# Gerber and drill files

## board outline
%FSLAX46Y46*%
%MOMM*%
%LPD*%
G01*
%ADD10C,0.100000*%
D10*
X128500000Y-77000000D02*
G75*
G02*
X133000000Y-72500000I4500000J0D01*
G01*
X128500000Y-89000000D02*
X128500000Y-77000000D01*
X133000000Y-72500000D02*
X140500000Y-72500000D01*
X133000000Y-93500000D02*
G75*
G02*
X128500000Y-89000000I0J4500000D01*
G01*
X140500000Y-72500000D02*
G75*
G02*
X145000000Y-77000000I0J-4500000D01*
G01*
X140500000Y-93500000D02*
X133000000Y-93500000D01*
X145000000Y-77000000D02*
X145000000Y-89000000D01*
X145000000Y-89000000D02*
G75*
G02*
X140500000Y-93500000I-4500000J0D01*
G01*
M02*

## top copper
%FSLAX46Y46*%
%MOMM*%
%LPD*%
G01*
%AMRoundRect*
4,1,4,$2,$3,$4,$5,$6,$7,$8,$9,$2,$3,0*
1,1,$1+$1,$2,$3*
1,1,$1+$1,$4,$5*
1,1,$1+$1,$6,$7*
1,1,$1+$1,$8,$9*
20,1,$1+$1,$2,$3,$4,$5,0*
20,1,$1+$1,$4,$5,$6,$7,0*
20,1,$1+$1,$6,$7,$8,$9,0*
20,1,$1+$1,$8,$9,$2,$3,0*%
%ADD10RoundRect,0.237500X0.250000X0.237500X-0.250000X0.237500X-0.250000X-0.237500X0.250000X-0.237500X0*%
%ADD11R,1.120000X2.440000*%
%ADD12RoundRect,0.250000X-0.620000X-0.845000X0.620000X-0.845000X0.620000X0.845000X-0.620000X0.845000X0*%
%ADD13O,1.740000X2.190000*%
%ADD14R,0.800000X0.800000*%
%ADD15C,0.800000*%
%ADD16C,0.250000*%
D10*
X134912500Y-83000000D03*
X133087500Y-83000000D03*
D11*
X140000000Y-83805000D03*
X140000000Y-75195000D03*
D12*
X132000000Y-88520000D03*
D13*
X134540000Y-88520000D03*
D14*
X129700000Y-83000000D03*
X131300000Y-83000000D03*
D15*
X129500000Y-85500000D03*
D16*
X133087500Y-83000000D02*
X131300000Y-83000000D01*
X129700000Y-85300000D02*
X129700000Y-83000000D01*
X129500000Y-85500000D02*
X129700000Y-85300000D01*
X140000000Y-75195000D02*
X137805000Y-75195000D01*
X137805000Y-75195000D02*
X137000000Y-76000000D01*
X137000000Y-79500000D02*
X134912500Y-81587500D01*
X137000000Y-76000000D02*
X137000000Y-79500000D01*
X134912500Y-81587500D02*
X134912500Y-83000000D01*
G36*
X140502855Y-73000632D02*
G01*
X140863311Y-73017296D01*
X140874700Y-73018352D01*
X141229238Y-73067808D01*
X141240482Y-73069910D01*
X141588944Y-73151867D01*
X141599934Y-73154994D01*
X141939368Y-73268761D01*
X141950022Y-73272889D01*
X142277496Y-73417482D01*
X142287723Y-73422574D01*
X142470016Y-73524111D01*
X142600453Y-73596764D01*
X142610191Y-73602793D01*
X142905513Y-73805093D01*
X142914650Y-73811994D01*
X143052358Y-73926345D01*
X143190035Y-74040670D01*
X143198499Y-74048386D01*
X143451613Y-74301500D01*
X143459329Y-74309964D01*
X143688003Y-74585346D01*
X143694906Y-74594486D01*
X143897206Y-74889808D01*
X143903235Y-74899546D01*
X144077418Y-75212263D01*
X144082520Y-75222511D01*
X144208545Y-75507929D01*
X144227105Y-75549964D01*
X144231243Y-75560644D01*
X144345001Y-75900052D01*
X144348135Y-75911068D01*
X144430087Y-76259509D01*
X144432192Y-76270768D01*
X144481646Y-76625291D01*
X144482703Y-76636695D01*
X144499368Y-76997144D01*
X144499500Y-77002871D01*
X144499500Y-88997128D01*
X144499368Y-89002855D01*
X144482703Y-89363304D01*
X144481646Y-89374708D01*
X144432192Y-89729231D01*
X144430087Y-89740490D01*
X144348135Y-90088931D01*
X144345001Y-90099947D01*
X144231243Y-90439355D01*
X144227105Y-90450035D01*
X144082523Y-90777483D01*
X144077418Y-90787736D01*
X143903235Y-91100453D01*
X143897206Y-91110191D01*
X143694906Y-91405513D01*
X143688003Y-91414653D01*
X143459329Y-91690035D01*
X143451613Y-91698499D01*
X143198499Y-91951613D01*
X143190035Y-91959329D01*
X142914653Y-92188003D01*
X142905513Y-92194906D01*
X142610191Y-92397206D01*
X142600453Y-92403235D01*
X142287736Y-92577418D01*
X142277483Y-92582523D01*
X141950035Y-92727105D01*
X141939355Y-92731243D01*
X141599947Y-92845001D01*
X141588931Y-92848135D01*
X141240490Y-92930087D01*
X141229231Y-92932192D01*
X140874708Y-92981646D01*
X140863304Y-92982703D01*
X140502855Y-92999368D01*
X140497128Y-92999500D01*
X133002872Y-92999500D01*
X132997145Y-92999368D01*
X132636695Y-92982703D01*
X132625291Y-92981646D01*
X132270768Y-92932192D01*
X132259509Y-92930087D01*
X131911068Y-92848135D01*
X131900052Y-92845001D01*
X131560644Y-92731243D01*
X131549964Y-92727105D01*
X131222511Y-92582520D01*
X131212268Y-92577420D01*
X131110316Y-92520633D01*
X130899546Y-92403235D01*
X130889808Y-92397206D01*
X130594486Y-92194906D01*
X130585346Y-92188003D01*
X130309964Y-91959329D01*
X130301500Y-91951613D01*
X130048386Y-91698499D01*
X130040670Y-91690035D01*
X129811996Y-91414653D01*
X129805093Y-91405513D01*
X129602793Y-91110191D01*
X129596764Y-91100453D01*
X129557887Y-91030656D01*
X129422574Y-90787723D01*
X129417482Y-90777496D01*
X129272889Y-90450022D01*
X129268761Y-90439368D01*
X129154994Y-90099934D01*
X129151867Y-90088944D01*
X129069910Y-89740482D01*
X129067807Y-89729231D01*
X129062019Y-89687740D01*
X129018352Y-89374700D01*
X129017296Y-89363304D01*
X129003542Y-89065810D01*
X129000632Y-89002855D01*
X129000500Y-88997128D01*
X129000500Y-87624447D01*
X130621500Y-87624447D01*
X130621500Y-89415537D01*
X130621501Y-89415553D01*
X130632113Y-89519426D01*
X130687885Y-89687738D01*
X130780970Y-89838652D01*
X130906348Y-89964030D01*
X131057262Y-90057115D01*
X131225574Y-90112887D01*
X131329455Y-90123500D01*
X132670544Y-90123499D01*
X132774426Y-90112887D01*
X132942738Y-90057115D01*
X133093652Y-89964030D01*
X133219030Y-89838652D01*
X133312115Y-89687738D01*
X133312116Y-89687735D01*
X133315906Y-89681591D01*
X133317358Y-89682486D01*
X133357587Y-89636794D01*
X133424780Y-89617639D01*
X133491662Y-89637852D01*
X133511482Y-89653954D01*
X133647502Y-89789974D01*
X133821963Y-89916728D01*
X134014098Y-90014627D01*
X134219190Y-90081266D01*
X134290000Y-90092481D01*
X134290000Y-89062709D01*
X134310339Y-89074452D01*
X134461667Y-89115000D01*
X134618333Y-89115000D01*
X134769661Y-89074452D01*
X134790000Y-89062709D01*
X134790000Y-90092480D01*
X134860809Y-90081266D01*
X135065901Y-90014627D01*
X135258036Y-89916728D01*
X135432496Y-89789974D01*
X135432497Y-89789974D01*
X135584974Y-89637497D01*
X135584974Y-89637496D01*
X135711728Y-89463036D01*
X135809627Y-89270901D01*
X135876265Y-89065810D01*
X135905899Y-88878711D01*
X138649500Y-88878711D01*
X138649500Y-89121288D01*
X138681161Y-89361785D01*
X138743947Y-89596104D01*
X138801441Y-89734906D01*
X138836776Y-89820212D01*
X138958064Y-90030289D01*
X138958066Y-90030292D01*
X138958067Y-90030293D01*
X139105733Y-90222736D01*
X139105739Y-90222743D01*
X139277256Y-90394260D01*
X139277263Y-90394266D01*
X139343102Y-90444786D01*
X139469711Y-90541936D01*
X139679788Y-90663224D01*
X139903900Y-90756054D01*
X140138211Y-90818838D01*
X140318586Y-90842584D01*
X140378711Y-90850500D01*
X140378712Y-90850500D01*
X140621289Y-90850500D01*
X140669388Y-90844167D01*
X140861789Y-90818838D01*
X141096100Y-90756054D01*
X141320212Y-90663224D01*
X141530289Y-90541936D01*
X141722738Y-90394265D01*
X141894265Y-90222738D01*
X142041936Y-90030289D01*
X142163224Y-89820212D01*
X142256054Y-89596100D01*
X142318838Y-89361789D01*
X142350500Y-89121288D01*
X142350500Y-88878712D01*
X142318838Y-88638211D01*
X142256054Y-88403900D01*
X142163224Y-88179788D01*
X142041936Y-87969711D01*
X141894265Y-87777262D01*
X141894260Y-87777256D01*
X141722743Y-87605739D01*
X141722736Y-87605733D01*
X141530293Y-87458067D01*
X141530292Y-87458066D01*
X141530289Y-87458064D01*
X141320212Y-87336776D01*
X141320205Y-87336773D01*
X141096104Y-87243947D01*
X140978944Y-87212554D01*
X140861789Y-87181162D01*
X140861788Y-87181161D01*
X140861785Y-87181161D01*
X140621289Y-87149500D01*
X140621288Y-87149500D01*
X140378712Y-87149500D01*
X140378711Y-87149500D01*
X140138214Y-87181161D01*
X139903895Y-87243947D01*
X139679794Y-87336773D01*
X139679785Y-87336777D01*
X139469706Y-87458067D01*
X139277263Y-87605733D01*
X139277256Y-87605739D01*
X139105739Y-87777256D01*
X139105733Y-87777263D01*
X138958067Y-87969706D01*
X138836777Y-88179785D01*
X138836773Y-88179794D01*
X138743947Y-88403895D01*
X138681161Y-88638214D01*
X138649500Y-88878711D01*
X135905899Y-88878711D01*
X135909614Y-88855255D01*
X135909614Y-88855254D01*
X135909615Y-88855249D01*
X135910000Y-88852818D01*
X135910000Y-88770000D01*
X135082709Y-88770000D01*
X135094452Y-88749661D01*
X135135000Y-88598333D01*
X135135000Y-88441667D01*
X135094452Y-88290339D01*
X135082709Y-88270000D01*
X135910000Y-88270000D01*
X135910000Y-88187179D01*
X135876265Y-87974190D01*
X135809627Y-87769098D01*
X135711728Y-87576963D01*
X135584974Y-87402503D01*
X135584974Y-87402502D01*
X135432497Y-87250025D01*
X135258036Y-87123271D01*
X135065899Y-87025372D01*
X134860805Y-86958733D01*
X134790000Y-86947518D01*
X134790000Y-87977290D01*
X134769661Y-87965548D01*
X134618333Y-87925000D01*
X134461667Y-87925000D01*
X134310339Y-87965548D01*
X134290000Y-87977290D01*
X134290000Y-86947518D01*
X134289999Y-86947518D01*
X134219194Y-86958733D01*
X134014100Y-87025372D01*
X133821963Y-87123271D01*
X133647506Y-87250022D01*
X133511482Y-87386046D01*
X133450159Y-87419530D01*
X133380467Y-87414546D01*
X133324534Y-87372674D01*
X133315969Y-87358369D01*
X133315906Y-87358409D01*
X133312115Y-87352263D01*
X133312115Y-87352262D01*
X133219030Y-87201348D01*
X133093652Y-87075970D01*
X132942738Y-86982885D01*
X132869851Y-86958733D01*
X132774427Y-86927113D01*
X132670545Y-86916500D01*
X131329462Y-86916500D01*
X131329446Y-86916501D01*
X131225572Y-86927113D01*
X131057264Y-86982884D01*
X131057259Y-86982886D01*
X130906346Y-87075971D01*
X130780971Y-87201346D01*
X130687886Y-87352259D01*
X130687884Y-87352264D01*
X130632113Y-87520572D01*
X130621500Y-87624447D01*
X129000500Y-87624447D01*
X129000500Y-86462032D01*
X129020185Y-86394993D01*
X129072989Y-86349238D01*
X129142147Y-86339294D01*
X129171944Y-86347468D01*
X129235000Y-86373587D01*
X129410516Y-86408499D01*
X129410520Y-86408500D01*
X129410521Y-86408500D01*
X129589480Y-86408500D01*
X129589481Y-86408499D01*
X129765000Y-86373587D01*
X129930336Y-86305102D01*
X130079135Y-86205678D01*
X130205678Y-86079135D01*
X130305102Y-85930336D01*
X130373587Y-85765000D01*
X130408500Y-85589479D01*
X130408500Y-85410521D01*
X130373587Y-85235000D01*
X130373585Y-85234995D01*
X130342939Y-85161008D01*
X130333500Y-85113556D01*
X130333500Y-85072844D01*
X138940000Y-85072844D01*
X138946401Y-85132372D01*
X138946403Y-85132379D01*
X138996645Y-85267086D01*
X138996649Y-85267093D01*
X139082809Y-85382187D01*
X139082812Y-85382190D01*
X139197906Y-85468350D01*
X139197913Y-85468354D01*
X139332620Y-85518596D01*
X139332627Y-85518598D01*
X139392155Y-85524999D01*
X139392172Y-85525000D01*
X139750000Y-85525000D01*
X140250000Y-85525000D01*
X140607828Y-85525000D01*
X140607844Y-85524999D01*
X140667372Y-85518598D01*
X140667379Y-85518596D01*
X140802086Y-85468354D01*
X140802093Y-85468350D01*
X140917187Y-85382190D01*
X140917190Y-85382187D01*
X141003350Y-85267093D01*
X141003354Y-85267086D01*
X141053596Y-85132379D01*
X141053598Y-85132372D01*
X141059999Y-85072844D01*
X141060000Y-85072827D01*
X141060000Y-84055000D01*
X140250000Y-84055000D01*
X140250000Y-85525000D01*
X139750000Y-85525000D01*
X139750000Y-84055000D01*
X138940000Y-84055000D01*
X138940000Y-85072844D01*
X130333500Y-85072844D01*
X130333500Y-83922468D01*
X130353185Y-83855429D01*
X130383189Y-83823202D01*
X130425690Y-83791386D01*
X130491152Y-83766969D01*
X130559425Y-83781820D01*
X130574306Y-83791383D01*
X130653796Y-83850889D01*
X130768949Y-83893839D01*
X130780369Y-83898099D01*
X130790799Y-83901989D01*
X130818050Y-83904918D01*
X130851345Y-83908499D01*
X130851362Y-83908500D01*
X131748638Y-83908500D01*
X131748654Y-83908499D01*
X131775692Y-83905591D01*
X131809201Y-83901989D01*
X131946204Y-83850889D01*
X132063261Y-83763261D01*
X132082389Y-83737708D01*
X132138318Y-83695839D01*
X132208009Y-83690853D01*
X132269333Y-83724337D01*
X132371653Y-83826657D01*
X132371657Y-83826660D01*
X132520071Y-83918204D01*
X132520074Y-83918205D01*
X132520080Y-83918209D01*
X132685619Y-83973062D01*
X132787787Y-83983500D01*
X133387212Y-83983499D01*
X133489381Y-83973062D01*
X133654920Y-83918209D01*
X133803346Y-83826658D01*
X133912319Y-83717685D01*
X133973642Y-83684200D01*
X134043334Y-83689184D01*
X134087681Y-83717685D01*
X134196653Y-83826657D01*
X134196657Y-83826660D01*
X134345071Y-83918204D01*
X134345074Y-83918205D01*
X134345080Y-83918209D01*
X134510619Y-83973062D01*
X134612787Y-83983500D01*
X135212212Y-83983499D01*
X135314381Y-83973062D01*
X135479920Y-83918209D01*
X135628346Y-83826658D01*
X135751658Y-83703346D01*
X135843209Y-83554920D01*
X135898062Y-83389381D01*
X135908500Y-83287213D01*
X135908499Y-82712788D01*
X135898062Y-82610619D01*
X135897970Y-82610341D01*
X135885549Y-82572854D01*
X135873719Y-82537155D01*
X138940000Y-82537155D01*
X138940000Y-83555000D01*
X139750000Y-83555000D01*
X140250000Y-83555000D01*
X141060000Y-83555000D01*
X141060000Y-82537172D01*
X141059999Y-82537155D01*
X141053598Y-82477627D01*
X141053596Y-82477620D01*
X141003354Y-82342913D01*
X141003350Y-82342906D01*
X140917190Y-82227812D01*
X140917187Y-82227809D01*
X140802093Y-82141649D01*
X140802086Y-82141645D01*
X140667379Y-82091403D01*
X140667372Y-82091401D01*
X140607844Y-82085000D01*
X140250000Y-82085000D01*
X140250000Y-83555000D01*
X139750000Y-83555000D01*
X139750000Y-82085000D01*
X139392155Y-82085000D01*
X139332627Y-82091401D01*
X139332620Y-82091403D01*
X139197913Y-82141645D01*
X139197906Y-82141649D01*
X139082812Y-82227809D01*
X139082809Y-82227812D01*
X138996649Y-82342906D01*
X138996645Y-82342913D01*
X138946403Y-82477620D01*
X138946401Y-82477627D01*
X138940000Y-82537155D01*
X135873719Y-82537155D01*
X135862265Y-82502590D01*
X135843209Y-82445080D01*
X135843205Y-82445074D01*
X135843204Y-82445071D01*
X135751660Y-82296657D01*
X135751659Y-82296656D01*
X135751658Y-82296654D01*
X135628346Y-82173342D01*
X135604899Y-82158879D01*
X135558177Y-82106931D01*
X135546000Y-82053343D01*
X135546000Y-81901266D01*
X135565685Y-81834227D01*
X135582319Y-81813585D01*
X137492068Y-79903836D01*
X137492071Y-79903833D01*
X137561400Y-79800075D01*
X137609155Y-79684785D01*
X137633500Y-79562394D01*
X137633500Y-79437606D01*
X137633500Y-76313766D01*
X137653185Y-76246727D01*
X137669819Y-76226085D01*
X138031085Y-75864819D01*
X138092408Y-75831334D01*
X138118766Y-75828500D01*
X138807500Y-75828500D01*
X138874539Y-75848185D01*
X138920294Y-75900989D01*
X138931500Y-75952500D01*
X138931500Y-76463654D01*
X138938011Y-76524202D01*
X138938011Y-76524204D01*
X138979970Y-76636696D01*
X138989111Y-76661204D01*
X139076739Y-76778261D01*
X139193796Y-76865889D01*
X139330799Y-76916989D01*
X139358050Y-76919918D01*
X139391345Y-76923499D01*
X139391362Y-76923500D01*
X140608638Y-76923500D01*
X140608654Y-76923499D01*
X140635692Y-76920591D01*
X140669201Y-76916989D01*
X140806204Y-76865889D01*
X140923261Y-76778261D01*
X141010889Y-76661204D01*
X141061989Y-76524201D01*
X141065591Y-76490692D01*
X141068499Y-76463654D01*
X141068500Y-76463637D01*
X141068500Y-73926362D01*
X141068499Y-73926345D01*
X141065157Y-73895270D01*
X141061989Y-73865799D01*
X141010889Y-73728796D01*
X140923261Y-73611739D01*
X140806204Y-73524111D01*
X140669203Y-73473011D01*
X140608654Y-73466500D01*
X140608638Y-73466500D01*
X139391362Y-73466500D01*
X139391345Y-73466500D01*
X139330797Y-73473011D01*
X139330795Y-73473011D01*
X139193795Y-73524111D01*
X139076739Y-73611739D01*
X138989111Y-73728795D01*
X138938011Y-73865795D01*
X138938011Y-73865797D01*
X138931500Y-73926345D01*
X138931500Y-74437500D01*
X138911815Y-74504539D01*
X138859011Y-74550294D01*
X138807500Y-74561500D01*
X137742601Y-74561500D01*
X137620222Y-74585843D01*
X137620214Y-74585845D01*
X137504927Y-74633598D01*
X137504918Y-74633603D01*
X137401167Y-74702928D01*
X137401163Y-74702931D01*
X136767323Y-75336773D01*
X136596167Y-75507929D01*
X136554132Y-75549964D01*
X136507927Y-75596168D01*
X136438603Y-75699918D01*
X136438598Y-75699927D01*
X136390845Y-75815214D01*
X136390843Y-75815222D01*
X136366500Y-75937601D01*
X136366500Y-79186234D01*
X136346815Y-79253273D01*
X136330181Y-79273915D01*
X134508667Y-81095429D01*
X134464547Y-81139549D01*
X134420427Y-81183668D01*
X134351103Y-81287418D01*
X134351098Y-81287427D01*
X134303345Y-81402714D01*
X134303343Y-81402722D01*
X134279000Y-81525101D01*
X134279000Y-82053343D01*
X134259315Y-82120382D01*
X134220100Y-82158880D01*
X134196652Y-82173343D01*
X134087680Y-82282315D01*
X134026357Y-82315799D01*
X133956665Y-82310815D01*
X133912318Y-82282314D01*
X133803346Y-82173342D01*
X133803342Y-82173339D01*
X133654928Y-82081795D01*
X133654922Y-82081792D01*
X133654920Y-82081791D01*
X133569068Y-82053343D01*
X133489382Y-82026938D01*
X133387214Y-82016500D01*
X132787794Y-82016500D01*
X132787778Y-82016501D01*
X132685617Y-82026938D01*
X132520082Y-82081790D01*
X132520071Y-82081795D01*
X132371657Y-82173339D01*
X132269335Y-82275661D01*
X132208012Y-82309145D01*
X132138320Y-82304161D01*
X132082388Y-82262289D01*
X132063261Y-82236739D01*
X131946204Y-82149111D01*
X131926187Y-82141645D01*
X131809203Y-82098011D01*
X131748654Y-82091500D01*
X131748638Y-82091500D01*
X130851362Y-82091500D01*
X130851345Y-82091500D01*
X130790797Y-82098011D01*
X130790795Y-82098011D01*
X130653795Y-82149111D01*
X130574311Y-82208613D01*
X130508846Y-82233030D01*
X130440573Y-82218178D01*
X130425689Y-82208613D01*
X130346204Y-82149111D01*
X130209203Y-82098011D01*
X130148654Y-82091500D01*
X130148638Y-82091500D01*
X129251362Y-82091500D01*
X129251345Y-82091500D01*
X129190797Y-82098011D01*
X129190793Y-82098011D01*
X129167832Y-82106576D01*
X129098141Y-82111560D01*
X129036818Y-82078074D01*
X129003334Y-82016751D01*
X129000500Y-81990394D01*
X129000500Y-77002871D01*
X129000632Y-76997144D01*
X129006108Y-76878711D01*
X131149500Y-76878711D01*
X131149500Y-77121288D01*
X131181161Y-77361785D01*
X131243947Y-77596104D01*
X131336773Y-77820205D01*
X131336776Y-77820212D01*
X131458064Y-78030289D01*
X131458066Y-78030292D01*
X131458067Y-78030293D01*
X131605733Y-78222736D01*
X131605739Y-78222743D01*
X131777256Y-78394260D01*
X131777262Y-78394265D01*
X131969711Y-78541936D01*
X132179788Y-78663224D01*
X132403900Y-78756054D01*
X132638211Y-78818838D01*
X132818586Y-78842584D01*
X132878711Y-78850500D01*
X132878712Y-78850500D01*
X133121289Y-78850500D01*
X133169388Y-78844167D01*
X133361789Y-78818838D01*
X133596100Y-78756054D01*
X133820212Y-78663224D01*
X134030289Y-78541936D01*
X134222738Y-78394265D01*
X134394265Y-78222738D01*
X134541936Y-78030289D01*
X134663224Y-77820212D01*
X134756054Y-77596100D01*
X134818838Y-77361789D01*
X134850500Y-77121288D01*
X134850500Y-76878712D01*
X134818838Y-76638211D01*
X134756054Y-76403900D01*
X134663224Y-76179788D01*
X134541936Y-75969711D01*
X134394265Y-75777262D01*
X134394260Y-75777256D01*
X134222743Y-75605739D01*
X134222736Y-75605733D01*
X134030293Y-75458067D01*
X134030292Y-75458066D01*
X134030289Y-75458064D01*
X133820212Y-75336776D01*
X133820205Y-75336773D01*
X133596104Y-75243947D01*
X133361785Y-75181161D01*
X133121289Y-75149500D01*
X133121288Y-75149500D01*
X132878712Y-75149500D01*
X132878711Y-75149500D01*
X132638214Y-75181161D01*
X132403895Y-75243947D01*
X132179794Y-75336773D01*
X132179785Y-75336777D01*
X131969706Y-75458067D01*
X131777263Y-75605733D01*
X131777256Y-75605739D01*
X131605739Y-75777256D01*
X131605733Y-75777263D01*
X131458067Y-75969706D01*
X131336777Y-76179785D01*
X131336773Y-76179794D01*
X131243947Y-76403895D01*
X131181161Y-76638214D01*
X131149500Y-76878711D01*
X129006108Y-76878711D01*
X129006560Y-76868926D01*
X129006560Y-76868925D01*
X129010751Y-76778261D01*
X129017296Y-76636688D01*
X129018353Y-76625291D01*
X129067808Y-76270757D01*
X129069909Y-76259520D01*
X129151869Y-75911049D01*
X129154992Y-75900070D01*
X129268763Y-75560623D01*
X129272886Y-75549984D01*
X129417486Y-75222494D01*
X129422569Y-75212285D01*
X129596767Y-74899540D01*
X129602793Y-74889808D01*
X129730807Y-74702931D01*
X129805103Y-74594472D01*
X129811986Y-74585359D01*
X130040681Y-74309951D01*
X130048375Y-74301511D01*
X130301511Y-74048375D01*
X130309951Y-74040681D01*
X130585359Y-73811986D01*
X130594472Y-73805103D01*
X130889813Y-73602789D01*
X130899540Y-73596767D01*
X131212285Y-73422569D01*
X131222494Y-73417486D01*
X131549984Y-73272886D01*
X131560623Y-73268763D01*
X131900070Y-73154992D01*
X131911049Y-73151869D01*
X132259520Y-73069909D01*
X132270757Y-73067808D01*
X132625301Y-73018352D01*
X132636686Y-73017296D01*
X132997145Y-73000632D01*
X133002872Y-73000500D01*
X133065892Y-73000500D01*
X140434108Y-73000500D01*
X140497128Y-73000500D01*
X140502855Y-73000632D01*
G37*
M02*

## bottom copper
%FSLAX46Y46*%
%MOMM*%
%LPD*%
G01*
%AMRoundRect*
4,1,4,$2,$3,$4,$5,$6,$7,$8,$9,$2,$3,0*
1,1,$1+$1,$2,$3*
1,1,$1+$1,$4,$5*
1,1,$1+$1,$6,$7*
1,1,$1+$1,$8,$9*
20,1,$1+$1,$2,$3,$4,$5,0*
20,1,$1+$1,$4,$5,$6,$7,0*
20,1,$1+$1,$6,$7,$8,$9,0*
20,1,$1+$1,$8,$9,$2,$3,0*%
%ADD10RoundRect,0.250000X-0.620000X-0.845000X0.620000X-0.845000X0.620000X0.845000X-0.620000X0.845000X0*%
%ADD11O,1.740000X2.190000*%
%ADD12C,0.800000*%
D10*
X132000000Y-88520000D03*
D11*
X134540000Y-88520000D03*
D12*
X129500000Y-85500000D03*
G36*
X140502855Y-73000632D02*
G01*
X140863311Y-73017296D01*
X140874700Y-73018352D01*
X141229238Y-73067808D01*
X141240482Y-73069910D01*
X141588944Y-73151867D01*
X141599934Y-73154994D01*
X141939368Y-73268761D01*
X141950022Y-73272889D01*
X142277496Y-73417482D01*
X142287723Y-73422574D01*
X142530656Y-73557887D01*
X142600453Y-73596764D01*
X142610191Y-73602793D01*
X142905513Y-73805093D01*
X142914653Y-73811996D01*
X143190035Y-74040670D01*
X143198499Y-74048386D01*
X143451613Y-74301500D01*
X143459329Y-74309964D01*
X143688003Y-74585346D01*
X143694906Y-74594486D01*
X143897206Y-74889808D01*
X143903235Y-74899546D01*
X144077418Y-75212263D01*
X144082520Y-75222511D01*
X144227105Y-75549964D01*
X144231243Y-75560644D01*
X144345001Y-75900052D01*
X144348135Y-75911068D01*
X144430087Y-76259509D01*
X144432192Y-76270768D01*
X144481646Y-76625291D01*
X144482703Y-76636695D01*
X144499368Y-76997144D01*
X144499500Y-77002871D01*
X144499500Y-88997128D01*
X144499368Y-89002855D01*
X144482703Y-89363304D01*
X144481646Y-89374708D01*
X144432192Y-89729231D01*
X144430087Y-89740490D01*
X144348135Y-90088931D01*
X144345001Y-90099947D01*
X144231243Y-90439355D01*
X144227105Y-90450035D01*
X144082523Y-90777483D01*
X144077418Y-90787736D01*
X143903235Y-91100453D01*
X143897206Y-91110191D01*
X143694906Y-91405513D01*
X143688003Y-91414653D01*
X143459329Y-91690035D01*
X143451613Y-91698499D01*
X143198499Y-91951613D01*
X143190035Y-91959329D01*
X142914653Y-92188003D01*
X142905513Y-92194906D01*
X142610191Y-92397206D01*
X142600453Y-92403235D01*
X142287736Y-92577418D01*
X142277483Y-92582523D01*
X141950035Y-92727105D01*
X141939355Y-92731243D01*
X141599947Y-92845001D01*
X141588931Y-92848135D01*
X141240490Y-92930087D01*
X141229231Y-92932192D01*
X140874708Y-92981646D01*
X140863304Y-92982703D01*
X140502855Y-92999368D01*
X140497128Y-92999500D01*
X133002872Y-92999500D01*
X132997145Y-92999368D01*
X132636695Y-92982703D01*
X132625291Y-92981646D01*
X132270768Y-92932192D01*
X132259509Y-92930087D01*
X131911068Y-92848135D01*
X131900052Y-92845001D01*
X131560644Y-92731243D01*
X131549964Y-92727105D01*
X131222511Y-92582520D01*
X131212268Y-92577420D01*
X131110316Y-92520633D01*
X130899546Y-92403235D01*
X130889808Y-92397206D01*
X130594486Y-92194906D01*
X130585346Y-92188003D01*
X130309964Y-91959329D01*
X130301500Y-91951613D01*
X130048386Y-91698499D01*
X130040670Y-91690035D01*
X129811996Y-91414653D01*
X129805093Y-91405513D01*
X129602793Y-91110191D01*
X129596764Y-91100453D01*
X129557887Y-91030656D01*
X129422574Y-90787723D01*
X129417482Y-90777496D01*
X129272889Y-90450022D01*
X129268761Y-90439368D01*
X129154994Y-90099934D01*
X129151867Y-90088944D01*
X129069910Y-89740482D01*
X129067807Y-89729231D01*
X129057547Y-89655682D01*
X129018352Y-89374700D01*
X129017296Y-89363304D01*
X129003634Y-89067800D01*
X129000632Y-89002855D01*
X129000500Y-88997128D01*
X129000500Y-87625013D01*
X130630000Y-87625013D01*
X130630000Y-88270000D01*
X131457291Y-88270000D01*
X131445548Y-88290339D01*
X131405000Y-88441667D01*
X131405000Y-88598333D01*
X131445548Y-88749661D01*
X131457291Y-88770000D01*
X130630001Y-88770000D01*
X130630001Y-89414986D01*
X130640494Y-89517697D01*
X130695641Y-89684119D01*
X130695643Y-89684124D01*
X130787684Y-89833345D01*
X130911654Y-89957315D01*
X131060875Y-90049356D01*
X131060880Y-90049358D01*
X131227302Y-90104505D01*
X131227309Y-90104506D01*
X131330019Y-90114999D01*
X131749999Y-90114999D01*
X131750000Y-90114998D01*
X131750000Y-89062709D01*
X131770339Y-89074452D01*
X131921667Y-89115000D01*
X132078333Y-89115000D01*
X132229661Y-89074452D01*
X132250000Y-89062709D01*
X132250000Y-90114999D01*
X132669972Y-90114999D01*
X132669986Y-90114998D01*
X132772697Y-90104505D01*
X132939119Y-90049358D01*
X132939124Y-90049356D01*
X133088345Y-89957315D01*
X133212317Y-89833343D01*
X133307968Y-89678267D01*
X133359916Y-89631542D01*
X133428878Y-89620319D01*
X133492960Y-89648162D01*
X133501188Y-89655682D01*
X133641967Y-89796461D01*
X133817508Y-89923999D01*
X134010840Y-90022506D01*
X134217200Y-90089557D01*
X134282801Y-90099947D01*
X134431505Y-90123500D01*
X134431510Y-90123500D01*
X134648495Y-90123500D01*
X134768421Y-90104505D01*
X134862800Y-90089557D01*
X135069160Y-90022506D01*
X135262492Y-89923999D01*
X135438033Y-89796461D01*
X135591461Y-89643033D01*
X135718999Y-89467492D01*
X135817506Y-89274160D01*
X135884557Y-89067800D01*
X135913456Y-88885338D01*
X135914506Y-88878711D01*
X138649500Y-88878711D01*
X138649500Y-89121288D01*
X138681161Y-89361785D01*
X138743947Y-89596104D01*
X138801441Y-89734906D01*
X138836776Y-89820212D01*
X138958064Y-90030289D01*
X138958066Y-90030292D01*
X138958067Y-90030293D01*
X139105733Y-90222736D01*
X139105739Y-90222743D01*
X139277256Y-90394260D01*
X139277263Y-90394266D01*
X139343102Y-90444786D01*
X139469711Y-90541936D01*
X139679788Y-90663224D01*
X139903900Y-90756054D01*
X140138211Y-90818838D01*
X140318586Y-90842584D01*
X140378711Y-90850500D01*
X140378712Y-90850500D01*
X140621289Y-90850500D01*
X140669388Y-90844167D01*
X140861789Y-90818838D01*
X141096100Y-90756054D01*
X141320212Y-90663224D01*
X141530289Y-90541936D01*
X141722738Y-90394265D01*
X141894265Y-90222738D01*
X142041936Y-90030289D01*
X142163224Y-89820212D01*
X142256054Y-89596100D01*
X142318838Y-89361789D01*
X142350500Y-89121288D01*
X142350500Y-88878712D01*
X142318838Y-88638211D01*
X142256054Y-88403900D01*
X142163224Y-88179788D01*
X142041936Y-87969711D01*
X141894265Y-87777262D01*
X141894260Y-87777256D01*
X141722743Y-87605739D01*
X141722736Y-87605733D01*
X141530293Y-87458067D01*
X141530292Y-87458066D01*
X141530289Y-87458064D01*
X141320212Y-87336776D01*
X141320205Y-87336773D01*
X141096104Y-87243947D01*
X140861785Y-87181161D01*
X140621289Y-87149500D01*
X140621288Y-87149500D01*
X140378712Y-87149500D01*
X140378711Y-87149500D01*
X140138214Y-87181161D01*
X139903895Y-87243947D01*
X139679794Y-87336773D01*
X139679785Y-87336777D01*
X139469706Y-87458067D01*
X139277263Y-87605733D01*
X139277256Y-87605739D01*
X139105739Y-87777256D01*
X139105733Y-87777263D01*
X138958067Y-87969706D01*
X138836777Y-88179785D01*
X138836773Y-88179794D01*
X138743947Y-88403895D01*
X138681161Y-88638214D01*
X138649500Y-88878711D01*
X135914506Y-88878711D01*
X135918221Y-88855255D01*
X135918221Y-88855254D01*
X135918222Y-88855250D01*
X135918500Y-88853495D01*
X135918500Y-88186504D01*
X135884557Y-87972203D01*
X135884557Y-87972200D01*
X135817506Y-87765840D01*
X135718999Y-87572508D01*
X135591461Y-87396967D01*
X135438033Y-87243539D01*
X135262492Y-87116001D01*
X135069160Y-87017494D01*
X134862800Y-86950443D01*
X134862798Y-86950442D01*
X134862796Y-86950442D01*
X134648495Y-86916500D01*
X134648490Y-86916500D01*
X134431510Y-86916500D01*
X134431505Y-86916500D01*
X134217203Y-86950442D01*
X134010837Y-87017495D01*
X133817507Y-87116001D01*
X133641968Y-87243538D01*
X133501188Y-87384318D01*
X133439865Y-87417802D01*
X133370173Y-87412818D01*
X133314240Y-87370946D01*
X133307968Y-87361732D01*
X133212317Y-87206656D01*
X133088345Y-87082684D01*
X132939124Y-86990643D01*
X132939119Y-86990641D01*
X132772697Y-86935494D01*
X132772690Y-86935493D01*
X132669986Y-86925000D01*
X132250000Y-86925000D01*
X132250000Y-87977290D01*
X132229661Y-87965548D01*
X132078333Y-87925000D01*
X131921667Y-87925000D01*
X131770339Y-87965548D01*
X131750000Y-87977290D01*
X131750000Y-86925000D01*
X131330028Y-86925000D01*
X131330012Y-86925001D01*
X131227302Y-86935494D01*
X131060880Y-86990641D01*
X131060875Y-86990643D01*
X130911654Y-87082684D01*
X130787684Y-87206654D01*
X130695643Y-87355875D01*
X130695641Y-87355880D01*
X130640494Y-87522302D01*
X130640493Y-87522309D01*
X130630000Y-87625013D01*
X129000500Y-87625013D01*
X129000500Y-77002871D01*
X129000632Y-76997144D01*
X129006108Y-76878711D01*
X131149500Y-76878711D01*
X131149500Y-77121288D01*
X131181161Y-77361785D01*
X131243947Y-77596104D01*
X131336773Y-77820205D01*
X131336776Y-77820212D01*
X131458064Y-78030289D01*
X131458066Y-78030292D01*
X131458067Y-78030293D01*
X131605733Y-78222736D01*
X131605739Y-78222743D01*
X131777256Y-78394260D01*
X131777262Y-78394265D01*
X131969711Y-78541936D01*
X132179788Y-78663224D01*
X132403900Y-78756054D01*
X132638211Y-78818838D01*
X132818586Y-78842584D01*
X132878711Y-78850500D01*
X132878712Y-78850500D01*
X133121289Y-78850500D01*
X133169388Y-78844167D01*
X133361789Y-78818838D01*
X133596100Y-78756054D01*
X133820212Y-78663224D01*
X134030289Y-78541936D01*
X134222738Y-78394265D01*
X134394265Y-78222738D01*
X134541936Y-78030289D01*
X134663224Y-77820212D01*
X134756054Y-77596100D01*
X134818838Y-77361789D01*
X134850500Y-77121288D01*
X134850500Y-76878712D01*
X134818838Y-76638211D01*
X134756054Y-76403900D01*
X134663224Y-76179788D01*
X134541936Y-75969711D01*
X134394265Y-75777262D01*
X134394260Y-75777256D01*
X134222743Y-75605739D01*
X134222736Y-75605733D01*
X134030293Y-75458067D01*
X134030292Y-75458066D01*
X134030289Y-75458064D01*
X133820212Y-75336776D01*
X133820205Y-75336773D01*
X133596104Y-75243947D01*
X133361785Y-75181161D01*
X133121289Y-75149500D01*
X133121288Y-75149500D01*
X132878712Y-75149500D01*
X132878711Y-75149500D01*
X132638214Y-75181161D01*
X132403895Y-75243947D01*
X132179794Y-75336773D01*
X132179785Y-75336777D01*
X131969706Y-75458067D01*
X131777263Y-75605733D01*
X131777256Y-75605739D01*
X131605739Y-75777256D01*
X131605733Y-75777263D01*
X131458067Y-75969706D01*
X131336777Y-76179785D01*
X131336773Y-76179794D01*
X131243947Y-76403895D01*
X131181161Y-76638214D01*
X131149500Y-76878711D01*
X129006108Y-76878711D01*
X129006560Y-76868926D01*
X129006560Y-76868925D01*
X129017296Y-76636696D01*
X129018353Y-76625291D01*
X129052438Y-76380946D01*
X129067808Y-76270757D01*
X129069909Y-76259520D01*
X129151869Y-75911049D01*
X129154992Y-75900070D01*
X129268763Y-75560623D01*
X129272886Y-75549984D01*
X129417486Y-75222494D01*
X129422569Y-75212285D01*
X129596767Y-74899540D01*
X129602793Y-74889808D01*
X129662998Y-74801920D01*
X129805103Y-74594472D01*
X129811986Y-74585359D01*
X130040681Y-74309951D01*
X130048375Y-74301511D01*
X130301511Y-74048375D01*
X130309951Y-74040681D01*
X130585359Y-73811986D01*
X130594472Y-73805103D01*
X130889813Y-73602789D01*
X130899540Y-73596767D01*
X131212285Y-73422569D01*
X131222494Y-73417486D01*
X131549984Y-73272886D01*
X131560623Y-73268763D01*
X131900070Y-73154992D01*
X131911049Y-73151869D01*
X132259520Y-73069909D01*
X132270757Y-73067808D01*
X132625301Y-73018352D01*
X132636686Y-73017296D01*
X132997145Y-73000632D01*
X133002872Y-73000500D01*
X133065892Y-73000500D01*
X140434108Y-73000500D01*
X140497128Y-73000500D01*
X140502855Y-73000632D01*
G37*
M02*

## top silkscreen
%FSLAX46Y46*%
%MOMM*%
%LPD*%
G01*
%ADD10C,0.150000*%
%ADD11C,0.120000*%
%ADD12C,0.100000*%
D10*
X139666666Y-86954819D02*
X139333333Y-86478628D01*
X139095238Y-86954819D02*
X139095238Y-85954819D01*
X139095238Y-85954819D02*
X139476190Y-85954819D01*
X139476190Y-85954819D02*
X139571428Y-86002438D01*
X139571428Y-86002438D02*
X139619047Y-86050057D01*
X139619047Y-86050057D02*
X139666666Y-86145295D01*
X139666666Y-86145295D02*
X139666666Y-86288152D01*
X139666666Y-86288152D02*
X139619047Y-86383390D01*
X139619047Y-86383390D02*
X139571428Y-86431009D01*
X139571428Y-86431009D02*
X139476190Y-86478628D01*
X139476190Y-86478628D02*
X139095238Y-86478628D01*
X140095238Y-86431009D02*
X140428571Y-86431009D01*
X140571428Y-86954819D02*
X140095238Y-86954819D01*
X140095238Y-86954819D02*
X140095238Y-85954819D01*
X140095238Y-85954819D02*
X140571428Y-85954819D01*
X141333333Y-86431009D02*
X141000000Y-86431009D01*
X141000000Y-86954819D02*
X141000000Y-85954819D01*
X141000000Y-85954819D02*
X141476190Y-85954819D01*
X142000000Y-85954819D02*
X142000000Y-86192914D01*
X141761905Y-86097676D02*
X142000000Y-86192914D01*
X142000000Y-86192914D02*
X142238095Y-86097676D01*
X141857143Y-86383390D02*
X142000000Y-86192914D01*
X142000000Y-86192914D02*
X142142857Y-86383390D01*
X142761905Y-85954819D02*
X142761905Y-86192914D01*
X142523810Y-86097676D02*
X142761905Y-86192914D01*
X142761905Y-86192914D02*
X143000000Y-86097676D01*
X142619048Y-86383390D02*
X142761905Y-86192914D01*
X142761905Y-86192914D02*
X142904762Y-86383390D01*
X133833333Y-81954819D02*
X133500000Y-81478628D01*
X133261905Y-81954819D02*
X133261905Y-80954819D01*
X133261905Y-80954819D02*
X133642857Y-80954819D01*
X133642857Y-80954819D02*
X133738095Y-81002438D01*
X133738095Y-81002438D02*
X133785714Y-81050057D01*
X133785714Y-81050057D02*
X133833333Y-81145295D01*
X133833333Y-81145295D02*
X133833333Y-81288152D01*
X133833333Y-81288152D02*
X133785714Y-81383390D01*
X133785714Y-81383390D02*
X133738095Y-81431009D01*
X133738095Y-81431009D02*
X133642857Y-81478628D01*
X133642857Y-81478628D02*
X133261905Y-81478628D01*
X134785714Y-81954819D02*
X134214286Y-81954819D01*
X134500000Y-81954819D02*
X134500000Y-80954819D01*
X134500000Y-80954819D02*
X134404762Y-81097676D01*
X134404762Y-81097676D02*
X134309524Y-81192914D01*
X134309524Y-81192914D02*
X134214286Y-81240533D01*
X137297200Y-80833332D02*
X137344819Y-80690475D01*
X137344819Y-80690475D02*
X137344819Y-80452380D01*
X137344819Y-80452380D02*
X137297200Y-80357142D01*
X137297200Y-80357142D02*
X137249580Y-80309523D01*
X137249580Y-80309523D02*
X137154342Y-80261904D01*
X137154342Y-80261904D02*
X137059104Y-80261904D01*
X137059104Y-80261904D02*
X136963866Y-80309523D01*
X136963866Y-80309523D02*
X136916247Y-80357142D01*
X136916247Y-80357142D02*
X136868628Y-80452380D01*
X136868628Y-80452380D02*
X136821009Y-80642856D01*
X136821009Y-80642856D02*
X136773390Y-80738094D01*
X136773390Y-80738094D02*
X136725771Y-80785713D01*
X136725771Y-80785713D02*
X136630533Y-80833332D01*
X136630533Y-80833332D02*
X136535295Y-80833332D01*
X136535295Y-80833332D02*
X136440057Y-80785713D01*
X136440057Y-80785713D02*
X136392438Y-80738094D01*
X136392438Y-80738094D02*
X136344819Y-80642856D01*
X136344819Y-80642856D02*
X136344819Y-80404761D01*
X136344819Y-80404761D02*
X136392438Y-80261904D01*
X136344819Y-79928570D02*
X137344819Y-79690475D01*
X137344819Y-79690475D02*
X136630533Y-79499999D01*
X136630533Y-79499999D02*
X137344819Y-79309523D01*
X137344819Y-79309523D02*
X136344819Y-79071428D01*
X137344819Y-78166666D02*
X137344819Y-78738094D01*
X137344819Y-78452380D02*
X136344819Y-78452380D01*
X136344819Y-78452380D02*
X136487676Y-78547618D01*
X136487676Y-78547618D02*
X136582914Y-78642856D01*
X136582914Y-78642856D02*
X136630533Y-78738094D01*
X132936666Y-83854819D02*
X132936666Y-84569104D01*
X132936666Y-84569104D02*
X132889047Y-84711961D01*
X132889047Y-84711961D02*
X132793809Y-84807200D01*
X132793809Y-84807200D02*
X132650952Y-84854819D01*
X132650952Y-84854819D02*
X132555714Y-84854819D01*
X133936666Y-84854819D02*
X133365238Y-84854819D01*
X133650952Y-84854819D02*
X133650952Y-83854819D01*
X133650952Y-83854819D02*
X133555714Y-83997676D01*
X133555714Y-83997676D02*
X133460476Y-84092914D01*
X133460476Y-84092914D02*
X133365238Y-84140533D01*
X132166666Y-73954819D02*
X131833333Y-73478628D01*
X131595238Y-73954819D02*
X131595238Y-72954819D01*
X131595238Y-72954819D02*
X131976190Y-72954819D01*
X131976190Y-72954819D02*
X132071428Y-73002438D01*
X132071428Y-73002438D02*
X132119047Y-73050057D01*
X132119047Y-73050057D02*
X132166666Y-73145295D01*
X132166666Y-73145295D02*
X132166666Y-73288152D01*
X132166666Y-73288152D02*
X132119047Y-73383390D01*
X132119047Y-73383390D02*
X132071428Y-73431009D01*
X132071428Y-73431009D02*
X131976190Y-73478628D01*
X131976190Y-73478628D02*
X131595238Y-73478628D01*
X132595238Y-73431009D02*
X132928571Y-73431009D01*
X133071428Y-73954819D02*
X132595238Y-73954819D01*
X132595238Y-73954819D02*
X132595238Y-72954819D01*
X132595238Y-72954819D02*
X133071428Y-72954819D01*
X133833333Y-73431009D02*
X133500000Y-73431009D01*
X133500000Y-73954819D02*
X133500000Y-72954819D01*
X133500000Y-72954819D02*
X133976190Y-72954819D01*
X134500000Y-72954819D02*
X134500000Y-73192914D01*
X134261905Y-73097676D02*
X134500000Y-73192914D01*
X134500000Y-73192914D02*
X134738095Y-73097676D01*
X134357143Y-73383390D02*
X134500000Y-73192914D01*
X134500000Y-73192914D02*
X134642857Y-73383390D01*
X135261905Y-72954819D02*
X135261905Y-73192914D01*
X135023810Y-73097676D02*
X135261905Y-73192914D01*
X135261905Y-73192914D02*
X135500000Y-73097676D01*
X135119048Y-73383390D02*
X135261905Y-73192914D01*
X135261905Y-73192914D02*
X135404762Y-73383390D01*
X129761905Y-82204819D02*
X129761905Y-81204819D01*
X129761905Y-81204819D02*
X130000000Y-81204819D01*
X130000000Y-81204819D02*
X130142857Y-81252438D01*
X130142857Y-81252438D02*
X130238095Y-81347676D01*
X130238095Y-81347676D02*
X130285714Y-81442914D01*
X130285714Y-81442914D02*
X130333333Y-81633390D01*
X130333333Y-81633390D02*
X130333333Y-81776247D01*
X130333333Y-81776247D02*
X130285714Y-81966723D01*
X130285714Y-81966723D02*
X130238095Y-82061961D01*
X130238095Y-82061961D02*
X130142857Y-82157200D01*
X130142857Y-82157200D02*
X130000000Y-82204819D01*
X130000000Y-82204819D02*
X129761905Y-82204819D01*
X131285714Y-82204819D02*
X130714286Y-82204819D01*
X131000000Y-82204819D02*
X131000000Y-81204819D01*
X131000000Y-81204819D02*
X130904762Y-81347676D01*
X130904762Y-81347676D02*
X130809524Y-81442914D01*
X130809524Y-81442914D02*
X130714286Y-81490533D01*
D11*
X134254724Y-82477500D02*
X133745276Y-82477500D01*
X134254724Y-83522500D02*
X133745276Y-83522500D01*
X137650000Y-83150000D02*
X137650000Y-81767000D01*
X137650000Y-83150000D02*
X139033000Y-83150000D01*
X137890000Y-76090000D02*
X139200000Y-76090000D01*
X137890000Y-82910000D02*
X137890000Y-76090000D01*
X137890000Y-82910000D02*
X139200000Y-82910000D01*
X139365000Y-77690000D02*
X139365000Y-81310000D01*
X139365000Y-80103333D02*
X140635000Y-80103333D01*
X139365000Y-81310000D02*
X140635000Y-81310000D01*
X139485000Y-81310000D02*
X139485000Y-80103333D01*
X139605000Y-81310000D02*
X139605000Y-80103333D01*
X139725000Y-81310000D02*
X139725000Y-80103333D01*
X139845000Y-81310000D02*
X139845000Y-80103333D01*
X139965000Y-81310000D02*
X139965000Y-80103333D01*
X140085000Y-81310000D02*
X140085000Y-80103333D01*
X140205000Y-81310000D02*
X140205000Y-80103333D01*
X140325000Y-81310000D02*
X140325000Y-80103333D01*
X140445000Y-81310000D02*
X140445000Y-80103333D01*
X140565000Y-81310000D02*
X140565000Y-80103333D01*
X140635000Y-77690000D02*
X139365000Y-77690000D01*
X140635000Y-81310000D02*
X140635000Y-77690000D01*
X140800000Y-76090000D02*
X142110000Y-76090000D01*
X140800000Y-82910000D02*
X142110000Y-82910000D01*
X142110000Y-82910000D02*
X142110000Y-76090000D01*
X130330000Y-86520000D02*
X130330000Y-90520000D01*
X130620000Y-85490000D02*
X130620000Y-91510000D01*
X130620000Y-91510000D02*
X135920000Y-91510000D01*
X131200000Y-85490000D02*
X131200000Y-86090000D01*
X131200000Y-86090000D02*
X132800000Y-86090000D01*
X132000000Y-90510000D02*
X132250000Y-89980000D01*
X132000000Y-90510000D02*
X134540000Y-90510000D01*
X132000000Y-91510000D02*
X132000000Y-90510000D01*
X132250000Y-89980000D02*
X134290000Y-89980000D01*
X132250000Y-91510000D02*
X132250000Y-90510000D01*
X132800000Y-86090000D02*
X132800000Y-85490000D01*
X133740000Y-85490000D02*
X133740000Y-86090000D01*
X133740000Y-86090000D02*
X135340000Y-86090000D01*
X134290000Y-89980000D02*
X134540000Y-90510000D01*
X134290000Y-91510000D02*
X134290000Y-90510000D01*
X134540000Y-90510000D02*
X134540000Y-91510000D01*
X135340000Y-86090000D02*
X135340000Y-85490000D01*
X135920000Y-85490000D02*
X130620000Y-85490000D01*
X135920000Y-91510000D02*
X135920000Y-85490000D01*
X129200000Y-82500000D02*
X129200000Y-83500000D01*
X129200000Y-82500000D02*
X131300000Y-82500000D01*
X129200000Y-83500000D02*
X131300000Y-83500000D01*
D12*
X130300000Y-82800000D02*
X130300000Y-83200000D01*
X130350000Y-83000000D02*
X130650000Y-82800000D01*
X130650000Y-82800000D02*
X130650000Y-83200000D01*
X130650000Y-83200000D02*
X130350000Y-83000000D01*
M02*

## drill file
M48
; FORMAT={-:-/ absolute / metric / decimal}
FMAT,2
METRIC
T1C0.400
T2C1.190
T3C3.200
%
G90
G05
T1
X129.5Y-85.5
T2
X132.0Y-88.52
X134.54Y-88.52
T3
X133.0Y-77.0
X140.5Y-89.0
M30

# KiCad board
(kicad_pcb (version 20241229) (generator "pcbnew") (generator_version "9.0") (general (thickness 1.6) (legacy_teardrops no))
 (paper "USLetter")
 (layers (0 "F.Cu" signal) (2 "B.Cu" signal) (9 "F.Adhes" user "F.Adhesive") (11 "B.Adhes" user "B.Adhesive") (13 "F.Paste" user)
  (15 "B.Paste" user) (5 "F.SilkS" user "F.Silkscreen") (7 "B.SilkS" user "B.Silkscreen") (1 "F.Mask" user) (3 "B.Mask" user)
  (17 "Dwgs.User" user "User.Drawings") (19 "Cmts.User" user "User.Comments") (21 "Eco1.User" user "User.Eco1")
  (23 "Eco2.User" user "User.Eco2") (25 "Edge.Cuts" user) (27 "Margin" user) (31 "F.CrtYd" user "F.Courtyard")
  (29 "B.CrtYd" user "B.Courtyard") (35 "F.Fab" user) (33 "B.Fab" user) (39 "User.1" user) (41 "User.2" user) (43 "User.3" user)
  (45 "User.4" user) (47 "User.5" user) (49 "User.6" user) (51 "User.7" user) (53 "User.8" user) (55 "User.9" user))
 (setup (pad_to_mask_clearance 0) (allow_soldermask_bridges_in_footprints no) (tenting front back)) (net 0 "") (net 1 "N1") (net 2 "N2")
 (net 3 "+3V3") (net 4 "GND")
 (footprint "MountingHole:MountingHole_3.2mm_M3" (layer "F.Cu") (at 140.5 89)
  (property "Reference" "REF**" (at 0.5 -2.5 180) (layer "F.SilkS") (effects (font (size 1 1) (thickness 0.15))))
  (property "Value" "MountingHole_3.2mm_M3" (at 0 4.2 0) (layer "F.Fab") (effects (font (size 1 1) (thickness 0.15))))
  (pad "" np_thru_hole circle (at 0 0) (size 3.2 3.2) (drill 3.2) (layers "*.Cu" "*.Mask")))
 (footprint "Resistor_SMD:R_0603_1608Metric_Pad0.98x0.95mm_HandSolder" (layer "F.Cu") (at 134 83 180)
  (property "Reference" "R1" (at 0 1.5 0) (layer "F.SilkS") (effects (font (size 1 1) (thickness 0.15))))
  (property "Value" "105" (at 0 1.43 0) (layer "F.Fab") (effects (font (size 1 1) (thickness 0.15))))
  (fp_line (start -0.254724 0.5225) (end 0.254724 0.5225) (stroke (width 0.12) (type solid)) (layer "F.SilkS"))
  (fp_line (start -0.254724 -0.5225) (end 0.254724 -0.5225) (stroke (width 0.12) (type solid)) (layer "F.SilkS"))
  (pad "1" smd roundrect (at -0.9125 0 180) (size 0.975 0.95) (layers "F.Cu" "F.Mask" "F.Paste") (roundrect_rratio 0.25) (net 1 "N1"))
  (pad "2" smd roundrect (at 0.9125 0 180) (size 0.975 0.95) (layers "F.Cu" "F.Mask" "F.Paste") (roundrect_rratio 0.25) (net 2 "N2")))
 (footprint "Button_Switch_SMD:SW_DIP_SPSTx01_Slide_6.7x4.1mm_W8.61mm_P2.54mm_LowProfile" (layer "F.Cu") (at 140 79.5 90)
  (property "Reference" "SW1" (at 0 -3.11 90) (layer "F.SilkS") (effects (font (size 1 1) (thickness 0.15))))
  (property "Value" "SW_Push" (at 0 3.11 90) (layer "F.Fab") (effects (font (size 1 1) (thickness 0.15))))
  (fp_line (start -3.65 -2.35) (end -2.267 -2.35) (stroke (width 0.12) (type solid)) (layer "F.SilkS"))
  (fp_line (start -3.65 -2.35) (end -3.65 -0.967) (stroke (width 0.12) (type solid)) (layer "F.SilkS"))
  (fp_line (start 3.41 -2.11) (end 3.41 -0.8) (stroke (width 0.12) (type solid)) (layer "F.SilkS"))
  (fp_line (start -3.41 -2.11) (end 3.41 -2.11) (stroke (width 0.12) (type solid)) (layer "F.SilkS"))
  (fp_line (start -3.41 -2.11) (end -3.41 -0.8) (stroke (width 0.12) (type solid)) (layer "F.SilkS"))
  (fp_line (start 1.81 -0.635) (end -1.81 -0.635) (stroke (width 0.12) (type solid)) (layer "F.SilkS"))
  (fp_line (start -0.603333 -0.635) (end -0.603333 0.635) (stroke (width 0.12) (type solid)) (layer "F.SilkS"))
  (fp_line (start -1.81 -0.635) (end -1.81 0.635) (stroke (width 0.12) (type solid)) (layer "F.SilkS"))
  (fp_line (start -1.81 -0.515) (end -0.603333 -0.515) (stroke (width 0.12) (type solid)) (layer "F.SilkS"))
  (fp_line (start -1.81 -0.395) (end -0.603333 -0.395) (stroke (width 0.12) (type solid)) (layer "F.SilkS"))
  (fp_line (start -1.81 -0.275) (end -0.603333 -0.275) (stroke (width 0.12) (type solid)) (layer "F.SilkS"))
  (fp_line (start -1.81 -0.155) (end -0.603333 -0.155) (stroke (width 0.12) (type solid)) (layer "F.SilkS"))
  (fp_line (start -1.81 -0.035) (end -0.603333 -0.035) (stroke (width 0.12) (type solid)) (layer "F.SilkS"))
  (fp_line (start -1.81 0.085) (end -0.603333 0.085) (stroke (width 0.12) (type solid)) (layer "F.SilkS"))
  (fp_line (start -1.81 0.205) (end -0.603333 0.205) (stroke (width 0.12) (type solid)) (layer "F.SilkS"))
  (fp_line (start -1.81 0.325) (end -0.603333 0.325) (stroke (width 0.12) (type solid)) (layer "F.SilkS"))
  (fp_line (start -1.81 0.445) (end -0.603333 0.445) (stroke (width 0.12) (type solid)) (layer "F.SilkS"))
  (fp_line (start -1.81 0.565) (end -0.603333 0.565) (stroke (width 0.12) (type solid)) (layer "F.SilkS"))
  (fp_line (start 1.81 0.635) (end 1.81 -0.635) (stroke (width 0.12) (type solid)) (layer "F.SilkS"))
  (fp_line (start -1.81 0.635) (end 1.81 0.635) (stroke (width 0.12) (type solid)) (layer "F.SilkS"))
  (fp_line (start 3.41 0.8) (end 3.41 2.11) (stroke (width 0.12) (type solid)) (layer "F.SilkS"))
  (fp_line (start -3.41 0.8) (end -3.41 2.11) (stroke (width 0.12) (type solid)) (layer "F.SilkS"))
  (fp_line (start -3.41 2.11) (end 3.41 2.11) (stroke (width 0.12) (type solid)) (layer "F.SilkS"))
  (pad "1" smd rect (at -4.305 0 90) (size 2.44 1.12) (layers "F.Cu" "F.Mask" "F.Paste") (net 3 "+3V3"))
  (pad "2" smd rect (at 4.305 0 90) (size 2.44 1.12) (layers "F.Cu" "F.Mask" "F.Paste") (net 1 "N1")))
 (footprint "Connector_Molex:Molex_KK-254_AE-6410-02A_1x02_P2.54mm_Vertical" (layer "F.Cu") (at 132 88.52)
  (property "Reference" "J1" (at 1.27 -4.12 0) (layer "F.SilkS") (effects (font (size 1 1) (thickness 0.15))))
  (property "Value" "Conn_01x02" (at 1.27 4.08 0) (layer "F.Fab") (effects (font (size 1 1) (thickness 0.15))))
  (fp_line (start -1.67 -2) (end -1.67 2) (stroke (width 0.12) (type solid)) (layer "F.SilkS"))
  (fp_line (start -1.38 -3.03) (end -1.38 2.99) (stroke (width 0.12) (type solid)) (layer "F.SilkS"))
  (fp_line (start -1.38 2.99) (end 3.92 2.99) (stroke (width 0.12) (type solid)) (layer "F.SilkS"))
  (fp_line (start -0.8 -3.03) (end -0.8 -2.43) (stroke (width 0.12) (type solid)) (layer "F.SilkS"))
  (fp_line (start -0.8 -2.43) (end 0.8 -2.43) (stroke (width 0.12) (type solid)) (layer "F.SilkS"))
  (fp_line (start 0 1.99) (end 0.25 1.46) (stroke (width 0.12) (type solid)) (layer "F.SilkS"))
  (fp_line (start 0 1.99) (end 2.54 1.99) (stroke (width 0.12) (type solid)) (layer "F.SilkS"))
  (fp_line (start 0 2.99) (end 0 1.99) (stroke (width 0.12) (type solid)) (layer "F.SilkS"))
  (fp_line (start 0.25 1.46) (end 2.29 1.46) (stroke (width 0.12) (type solid)) (layer "F.SilkS"))
  (fp_line (start 0.25 2.99) (end 0.25 1.99) (stroke (width 0.12) (type solid)) (layer "F.SilkS"))
  (fp_line (start 0.8 -2.43) (end 0.8 -3.03) (stroke (width 0.12) (type solid)) (layer "F.SilkS"))
  (fp_line (start 1.74 -3.03) (end 1.74 -2.43) (stroke (width 0.12) (type solid)) (layer "F.SilkS"))
  (fp_line (start 1.74 -2.43) (end 3.34 -2.43) (stroke (width 0.12) (type solid)) (layer "F.SilkS"))
  (fp_line (start 2.29 1.46) (end 2.54 1.99) (stroke (width 0.12) (type solid)) (layer "F.SilkS"))
  (fp_line (start 2.29 2.99) (end 2.29 1.99) (stroke (width 0.12) (type solid)) (layer "F.SilkS"))
  (fp_line (start 2.54 1.99) (end 2.54 2.99) (stroke (width 0.12) (type solid)) (layer "F.SilkS"))
  (fp_line (start 3.34 -2.43) (end 3.34 -3.03) (stroke (width 0.12) (type solid)) (layer "F.SilkS"))
  (fp_line (start 3.92 -3.03) (end -1.38 -3.03) (stroke (width 0.12) (type solid)) (layer "F.SilkS"))
  (fp_line (start 3.92 2.99) (end 3.92 -3.03) (stroke (width 0.12) (type solid)) (layer "F.SilkS"))
  (pad "1" thru_hole roundrect (at 0 0) (size 1.74 2.19) (drill 1.19) (layers "*.Cu" "*.Mask") (remove_unused_layers no)
   (roundrect_rratio 0.143678) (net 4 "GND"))
  (pad "2" thru_hole oval (at 2.54 0) (size 1.74 2.19) (drill 1.19) (layers "*.Cu" "*.Mask") (remove_unused_layers no) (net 3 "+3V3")))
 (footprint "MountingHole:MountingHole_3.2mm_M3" (layer "F.Cu") (at 133 77)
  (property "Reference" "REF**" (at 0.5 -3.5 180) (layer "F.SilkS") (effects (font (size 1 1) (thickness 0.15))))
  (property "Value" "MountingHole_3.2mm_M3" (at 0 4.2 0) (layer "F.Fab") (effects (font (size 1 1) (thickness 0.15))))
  (pad "" np_thru_hole circle (at 0 0) (size 3.2 3.2) (drill 3.2) (layers "*.Cu" "*.Mask")))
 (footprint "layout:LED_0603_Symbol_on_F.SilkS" (layer "F.Cu") (at 130.5 83)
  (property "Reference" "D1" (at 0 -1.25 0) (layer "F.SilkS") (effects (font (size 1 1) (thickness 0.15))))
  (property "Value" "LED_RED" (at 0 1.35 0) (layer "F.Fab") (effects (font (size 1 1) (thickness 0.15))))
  (fp_line (start -1.3 -0.5) (end -1.3 0.5) (stroke (width 0.12) (type solid)) (layer "F.SilkS"))
  (fp_line (start -1.3 -0.5) (end 0.8 -0.5) (stroke (width 0.12) (type solid)) (layer "F.SilkS"))
  (fp_line (start -1.3 0.5) (end 0.8 0.5) (stroke (width 0.12) (type solid)) (layer "F.SilkS"))
  (fp_line (start -0.2 -0.2) (end -0.2 0.2) (stroke (width 0.1) (type solid)) (layer "F.SilkS"))
  (fp_line (start -0.15 0) (end 0.15 -0.2) (stroke (width 0.1) (type solid)) (layer "F.SilkS"))
  (fp_line (start 0.15 -0.2) (end 0.15 0.2) (stroke (width 0.1) (type solid)) (layer "F.SilkS"))
  (fp_line (start 0.15 0.2) (end -0.15 0) (stroke (width 0.1) (type solid)) (layer "F.SilkS"))
  (pad "1" smd rect (at -0.8 0 180) (size 0.8 0.8) (layers "F.Cu" "F.Mask" "F.Paste") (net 4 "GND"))
  (pad "2" smd rect (at 0.8 0 180) (size 0.8 0.8) (layers "F.Cu" "F.Mask" "F.Paste") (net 2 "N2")))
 (gr_arc (start 128.5 77) (mid 129.818019 73.818019) (end 133 72.5) (stroke (width 0.1) (type default)) (layer "Edge.Cuts"))
 (gr_line (start 128.5 89) (end 128.5 77) (stroke (width 0.1) (type default)) (layer "Edge.Cuts"))
 (gr_line (start 133 72.5) (end 140.5 72.5) (stroke (width 0.1) (type default)) (layer "Edge.Cuts"))
 (gr_arc (start 133 93.5) (mid 129.818019 92.181981) (end 128.5 89) (stroke (width 0.1) (type default)) (layer "Edge.Cuts"))
 (gr_arc (start 140.5 72.5) (mid 143.681981 73.818019) (end 145 77) (stroke (width 0.1) (type default)) (layer "Edge.Cuts"))
 (gr_line (start 140.5 93.5) (end 133 93.5) (stroke (width 0.1) (type default)) (layer "Edge.Cuts"))
 (gr_line (start 145 77) (end 145 89) (stroke (width 0.1) (type default)) (layer "Edge.Cuts"))
 (gr_arc (start 145 89) (mid 143.681981 92.181981) (end 140.5 93.5) (stroke (width 0.1) (type default)) (layer "Edge.Cuts"))
 (segment (start 133.0875 83) (end 131.3 83) (width 0.25) (layer "F.Cu") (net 2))
 (segment (start 129.7 85.3) (end 129.7 83) (width 0.25) (layer "F.Cu") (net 4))
 (segment (start 129.5 85.5) (end 129.7 85.3) (width 0.25) (layer "F.Cu") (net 4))
 (via (at 129.5 85.5) (size 0.8) (drill 0.4) (layers "F.Cu" "B.Cu") (free yes) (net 4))
 (segment (start 140 75.195) (end 137.805 75.195) (width 0.25) (layer "F.Cu") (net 1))
 (segment (start 137.805 75.195) (end 137 76) (width 0.25) (layer "F.Cu") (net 1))
 (segment (start 137 79.5) (end 134.9125 81.5875) (width 0.25) (layer "F.Cu") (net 1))
 (segment (start 137 76) (end 137 79.5) (width 0.25) (layer "F.Cu") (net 1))
 (segment (start 134.9125 81.5875) (end 134.9125 83) (width 0.25) (layer "F.Cu") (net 1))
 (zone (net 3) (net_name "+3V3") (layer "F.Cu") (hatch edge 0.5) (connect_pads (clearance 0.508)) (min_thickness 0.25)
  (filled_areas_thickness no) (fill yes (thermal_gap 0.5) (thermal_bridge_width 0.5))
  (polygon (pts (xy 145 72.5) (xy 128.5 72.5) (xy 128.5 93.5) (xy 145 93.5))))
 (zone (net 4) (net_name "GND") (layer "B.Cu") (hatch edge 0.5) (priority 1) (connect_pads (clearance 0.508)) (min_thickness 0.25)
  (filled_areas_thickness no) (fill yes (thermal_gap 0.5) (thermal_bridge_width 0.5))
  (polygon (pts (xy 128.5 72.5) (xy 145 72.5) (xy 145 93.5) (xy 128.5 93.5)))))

